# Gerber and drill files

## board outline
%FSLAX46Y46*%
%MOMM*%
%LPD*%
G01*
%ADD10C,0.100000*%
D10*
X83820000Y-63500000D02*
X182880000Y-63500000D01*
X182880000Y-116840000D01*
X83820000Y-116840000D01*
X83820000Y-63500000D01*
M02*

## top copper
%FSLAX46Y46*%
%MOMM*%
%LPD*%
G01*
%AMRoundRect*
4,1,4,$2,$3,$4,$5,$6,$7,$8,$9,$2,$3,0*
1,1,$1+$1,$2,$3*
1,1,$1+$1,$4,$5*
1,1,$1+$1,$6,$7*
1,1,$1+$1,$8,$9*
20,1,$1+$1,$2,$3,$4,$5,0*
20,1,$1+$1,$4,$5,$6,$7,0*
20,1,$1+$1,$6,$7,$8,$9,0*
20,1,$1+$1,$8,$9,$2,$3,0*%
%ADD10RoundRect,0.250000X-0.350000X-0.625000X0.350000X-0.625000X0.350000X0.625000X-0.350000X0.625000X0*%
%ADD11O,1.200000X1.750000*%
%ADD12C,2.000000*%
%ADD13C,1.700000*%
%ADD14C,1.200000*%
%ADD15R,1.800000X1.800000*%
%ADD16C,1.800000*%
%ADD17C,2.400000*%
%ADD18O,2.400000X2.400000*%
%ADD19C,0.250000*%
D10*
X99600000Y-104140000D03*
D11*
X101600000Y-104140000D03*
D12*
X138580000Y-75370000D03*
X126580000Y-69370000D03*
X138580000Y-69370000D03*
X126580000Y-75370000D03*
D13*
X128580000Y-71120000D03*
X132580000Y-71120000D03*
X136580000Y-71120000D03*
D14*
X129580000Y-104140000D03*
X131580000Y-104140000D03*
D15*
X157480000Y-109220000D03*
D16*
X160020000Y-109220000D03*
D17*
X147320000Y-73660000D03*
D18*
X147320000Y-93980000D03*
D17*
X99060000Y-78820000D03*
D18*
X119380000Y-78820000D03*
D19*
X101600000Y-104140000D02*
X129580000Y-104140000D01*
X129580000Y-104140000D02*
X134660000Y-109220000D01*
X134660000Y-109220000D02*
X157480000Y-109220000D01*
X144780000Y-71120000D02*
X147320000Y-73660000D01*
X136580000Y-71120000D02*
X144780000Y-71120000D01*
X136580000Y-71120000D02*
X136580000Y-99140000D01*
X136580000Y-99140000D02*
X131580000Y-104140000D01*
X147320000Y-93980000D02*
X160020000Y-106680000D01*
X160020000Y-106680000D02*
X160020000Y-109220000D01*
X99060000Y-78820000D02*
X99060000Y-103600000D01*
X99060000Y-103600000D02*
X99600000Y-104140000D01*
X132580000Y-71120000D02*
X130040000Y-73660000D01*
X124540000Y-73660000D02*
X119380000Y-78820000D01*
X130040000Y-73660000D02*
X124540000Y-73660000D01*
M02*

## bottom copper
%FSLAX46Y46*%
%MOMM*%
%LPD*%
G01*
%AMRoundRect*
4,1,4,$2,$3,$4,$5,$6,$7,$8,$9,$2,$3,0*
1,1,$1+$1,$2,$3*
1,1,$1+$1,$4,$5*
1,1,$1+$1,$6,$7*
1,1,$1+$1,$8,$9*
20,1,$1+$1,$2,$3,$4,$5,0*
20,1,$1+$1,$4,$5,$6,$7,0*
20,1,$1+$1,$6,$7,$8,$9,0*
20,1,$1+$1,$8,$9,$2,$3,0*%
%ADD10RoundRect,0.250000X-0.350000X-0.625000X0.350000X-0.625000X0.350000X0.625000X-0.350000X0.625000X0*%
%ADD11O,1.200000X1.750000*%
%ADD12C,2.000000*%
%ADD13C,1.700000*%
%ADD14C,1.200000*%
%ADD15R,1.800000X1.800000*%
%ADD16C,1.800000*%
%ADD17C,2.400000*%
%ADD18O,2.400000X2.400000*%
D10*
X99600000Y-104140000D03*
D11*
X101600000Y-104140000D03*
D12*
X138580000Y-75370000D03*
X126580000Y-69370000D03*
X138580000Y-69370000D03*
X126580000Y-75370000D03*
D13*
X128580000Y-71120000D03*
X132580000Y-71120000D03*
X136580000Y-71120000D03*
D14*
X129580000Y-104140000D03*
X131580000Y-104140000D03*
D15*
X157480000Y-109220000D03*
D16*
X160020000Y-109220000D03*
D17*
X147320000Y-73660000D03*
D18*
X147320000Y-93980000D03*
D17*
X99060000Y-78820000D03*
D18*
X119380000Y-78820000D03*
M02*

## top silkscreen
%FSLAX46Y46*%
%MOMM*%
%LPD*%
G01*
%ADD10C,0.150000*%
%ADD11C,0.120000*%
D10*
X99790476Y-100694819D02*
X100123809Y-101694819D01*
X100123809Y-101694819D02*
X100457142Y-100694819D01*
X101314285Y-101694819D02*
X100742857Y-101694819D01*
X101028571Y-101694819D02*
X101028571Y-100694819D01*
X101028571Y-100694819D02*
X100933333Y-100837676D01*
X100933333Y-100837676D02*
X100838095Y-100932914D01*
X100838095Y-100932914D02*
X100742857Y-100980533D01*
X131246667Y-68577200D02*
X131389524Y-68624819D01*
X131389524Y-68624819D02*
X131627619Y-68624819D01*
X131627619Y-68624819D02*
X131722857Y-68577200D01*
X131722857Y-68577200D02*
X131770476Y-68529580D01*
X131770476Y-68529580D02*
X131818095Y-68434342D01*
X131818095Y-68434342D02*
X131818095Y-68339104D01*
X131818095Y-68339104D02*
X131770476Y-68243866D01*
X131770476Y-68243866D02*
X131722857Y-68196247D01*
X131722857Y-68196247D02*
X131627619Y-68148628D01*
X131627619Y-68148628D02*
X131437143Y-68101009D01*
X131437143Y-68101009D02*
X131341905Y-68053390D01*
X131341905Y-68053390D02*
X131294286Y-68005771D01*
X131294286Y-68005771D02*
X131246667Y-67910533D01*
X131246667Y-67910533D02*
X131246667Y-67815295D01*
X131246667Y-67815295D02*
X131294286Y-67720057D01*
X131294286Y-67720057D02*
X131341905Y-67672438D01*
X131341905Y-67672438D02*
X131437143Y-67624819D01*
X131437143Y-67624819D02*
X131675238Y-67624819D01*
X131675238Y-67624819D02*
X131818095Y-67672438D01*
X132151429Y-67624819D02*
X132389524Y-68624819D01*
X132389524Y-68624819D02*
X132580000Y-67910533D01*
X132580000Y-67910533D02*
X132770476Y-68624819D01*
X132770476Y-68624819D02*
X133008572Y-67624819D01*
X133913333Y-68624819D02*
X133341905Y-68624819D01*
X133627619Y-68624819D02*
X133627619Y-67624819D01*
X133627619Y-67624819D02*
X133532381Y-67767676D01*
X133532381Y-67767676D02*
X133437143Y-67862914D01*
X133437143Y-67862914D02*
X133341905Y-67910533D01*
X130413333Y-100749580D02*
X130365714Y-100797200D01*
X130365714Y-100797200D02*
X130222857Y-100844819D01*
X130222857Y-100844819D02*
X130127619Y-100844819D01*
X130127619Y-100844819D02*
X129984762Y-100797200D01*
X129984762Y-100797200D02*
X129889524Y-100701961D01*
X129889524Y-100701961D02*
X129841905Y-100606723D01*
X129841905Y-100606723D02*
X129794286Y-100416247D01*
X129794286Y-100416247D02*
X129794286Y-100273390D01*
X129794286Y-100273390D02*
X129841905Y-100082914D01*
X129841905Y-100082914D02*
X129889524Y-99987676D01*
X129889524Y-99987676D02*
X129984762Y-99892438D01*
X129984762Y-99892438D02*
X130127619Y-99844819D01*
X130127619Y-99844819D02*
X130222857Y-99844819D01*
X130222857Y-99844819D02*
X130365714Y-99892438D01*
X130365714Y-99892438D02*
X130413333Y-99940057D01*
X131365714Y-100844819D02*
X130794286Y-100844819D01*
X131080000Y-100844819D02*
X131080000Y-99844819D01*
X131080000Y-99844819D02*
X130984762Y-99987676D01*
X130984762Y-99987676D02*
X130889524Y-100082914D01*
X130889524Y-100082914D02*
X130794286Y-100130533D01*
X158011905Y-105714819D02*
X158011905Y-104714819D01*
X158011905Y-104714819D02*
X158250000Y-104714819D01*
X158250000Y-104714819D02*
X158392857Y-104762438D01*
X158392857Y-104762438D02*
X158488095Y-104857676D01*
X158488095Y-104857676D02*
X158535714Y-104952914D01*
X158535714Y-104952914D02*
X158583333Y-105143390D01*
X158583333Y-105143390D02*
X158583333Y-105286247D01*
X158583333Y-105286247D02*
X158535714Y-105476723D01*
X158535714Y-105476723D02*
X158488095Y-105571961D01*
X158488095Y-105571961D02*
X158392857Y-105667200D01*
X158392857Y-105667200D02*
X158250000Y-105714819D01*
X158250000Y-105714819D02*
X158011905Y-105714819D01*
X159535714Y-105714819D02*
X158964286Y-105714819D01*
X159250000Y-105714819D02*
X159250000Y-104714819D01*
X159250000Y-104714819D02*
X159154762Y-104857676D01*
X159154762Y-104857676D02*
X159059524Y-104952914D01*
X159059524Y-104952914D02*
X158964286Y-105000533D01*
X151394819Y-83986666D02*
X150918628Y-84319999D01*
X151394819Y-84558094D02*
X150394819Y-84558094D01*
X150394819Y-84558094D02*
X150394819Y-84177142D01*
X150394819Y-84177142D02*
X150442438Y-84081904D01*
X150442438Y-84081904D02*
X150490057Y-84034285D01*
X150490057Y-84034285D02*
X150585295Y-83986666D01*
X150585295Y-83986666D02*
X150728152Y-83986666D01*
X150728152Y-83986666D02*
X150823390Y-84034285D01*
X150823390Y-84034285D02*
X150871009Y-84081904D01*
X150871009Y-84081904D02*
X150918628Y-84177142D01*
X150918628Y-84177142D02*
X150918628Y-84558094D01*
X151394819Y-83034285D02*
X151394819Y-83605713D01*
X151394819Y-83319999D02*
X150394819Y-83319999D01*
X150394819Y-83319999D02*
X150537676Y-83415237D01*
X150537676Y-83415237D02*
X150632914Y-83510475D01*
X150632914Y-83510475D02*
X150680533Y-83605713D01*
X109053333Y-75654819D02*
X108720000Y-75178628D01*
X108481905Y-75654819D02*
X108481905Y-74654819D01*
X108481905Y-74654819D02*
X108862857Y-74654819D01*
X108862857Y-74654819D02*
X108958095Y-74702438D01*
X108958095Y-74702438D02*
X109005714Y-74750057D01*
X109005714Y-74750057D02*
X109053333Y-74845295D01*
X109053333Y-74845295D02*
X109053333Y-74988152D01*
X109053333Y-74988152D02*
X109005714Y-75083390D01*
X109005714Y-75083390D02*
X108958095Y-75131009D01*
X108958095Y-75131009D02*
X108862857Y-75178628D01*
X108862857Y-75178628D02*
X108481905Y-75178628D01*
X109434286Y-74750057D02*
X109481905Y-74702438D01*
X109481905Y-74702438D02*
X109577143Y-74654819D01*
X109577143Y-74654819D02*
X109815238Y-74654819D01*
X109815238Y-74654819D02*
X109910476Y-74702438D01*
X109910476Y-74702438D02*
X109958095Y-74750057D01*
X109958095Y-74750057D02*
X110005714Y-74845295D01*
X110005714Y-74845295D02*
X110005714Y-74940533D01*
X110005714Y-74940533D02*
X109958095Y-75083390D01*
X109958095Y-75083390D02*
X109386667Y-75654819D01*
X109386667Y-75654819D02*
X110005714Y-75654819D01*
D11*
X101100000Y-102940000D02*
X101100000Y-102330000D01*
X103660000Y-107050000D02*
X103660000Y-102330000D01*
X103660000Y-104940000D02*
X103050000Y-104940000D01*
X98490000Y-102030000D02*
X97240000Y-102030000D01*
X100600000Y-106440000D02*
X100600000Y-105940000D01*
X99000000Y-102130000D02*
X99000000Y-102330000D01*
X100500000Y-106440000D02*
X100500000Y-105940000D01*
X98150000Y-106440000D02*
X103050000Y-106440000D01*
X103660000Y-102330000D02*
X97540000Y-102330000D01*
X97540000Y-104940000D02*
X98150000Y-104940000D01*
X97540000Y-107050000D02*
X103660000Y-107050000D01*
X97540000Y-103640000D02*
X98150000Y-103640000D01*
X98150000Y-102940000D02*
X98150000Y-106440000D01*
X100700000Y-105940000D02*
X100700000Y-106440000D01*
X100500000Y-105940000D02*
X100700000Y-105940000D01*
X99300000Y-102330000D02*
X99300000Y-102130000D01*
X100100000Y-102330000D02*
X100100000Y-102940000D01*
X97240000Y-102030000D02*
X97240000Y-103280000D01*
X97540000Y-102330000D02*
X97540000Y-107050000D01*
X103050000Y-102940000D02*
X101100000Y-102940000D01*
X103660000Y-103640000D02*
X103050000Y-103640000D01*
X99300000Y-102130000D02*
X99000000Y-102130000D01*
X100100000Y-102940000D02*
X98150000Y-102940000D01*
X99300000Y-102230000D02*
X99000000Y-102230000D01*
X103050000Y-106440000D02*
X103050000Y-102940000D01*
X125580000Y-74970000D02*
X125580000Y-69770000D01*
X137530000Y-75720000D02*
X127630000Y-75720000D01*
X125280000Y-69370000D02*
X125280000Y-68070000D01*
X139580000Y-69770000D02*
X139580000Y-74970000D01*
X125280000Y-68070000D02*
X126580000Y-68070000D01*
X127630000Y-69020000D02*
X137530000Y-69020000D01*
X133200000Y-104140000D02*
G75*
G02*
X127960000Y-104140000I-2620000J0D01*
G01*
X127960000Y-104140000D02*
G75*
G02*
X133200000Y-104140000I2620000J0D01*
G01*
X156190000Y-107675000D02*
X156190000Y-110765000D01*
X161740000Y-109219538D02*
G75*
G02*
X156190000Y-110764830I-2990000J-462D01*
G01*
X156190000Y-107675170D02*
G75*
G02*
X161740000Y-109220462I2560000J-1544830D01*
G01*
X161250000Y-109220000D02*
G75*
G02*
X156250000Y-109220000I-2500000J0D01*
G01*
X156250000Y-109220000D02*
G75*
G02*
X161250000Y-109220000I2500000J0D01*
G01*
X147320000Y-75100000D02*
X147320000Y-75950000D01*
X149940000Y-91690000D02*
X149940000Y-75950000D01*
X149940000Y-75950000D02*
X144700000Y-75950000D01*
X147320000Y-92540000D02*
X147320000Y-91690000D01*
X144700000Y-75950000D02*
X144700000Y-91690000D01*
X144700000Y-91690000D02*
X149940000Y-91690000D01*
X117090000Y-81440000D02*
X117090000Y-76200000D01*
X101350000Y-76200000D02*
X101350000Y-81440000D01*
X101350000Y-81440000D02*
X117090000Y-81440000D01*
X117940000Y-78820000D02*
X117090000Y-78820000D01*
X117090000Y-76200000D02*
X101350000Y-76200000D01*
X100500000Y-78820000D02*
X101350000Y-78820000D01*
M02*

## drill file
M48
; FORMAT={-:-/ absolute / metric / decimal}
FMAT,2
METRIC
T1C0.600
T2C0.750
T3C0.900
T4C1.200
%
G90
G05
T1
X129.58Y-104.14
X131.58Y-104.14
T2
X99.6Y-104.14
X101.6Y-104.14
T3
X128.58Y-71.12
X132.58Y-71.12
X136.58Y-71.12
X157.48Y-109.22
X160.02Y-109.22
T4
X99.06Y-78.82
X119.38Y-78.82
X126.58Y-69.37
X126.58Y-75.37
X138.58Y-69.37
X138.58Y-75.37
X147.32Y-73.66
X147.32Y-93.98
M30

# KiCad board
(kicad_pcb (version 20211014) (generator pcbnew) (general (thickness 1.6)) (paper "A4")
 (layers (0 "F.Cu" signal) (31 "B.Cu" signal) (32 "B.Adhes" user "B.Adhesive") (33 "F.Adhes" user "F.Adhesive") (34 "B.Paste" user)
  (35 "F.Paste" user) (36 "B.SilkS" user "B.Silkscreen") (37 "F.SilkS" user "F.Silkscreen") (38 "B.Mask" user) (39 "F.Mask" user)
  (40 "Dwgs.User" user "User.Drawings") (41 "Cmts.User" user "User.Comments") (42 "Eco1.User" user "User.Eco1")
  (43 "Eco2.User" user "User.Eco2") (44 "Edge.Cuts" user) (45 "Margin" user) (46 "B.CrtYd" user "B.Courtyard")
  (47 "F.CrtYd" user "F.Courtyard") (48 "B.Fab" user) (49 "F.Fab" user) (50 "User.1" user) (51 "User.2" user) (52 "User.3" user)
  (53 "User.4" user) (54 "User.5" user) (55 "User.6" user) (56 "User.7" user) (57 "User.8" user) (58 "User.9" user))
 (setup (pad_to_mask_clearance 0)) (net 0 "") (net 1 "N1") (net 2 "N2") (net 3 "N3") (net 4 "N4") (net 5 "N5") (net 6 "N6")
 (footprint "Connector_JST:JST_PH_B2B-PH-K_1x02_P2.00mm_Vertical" (layer "F.Cu") (at 99.6 104.14)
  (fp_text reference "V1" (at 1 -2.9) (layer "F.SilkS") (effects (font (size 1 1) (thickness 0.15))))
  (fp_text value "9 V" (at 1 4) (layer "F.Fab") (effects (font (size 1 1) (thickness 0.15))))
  (fp_line (start 1.5 -1.2) (end 1.5 -1.81) (layer "F.SilkS") (width 0.12))
  (fp_line (start 4.06 2.91) (end 4.06 -1.81) (layer "F.SilkS") (width 0.12))
  (fp_line (start 4.06 0.8) (end 3.45 0.8) (layer "F.SilkS") (width 0.12))
  (fp_line (start -1.11 -2.11) (end -2.36 -2.11) (layer "F.SilkS") (width 0.12))
  (fp_line (start 1 2.3) (end 1 1.8) (layer "F.SilkS") (width 0.12))
  (fp_line (start -0.6 -2.01) (end -0.6 -1.81) (layer "F.SilkS") (width 0.12))
  (fp_line (start 0.9 2.3) (end 0.9 1.8) (layer "F.SilkS") (width 0.12))
  (fp_line (start -1.45 2.3) (end 3.45 2.3) (layer "F.SilkS") (width 0.12))
  (fp_line (start 4.06 -1.81) (end -2.06 -1.81) (layer "F.SilkS") (width 0.12))
  (fp_line (start -2.06 0.8) (end -1.45 0.8) (layer "F.SilkS") (width 0.12))
  (fp_line (start -2.06 2.91) (end 4.06 2.91) (layer "F.SilkS") (width 0.12))
  (fp_line (start -2.06 -0.5) (end -1.45 -0.5) (layer "F.SilkS") (width 0.12))
  (fp_line (start -1.45 -1.2) (end -1.45 2.3) (layer "F.SilkS") (width 0.12))
  (fp_line (start 1.1 1.8) (end 1.1 2.3) (layer "F.SilkS") (width 0.12))
  (fp_line (start 0.9 1.8) (end 1.1 1.8) (layer "F.SilkS") (width 0.12))
  (fp_line (start -0.3 -1.81) (end -0.3 -2.01) (layer "F.SilkS") (width 0.12))
  (fp_line (start 0.5 -1.81) (end 0.5 -1.2) (layer "F.SilkS") (width 0.12))
  (fp_line (start -2.36 -2.11) (end -2.36 -0.86) (layer "F.SilkS") (width 0.12))
  (fp_line (start -2.06 -1.81) (end -2.06 2.91) (layer "F.SilkS") (width 0.12))
  (fp_line (start 3.45 -1.2) (end 1.5 -1.2) (layer "F.SilkS") (width 0.12))
  (fp_line (start 4.06 -0.5) (end 3.45 -0.5) (layer "F.SilkS") (width 0.12))
  (fp_line (start -0.3 -2.01) (end -0.6 -2.01) (layer "F.SilkS") (width 0.12))
  (fp_line (start 0.5 -1.2) (end -1.45 -1.2) (layer "F.SilkS") (width 0.12))
  (fp_line (start -0.3 -1.91) (end -0.6 -1.91) (layer "F.SilkS") (width 0.12))
  (fp_line (start 3.45 2.3) (end 3.45 -1.2) (layer "F.SilkS") (width 0.12))
  (pad "1" thru_hole roundrect (at 0 0) (size 1.2 1.75) (drill 0.75) (layers *.Cu *.Mask) (roundrect_rratio 0.208333) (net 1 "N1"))
  (pad "2" thru_hole oval (at 2 0) (size 1.2 1.75) (drill 0.75) (layers *.Cu *.Mask) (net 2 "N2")))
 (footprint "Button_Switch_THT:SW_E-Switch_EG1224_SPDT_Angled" (layer "F.Cu") (at 128.58 71.12)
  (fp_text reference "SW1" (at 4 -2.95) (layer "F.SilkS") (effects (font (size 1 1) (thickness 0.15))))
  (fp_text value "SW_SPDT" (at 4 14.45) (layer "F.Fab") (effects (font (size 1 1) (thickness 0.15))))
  (fp_line (start -3 3.85) (end -3 -1.35) (layer "F.SilkS") (width 0.12))
  (fp_line (start 8.95 4.6) (end -0.95 4.6) (layer "F.SilkS") (width 0.12))
  (fp_line (start -3.3 -1.75) (end -3.3 -3.05) (layer "F.SilkS") (width 0.12))
  (fp_line (start 11 -1.35) (end 11 3.85) (layer "F.SilkS") (width 0.12))
  (fp_line (start -3.3 -3.05) (end -2 -3.05) (layer "F.SilkS") (width 0.12))
  (fp_line (start -0.95 -2.1) (end 8.95 -2.1) (layer "F.SilkS") (width 0.12))
  (pad "" thru_hole circle (at 10 4.25) (size 2 2) (drill 1.2) (layers *.Cu *.Mask))
  (pad "" thru_hole circle (at -2 -1.75) (size 2 2) (drill 1.2) (layers *.Cu *.Mask))
  (pad "" thru_hole circle (at 10 -1.75) (size 2 2) (drill 1.2) (layers *.Cu *.Mask))
  (pad "" thru_hole circle (at -2 4.25) (size 2 2) (drill 1.2) (layers *.Cu *.Mask))
  (pad "1" thru_hole circle (at 0 0) (size 1.7 1.7) (drill 0.9) (layers *.Cu *.Mask) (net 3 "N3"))
  (pad "2" thru_hole circle (at 4 0) (size 1.7 1.7) (drill 0.9) (layers *.Cu *.Mask) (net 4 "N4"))
  (pad "3" thru_hole circle (at 8 0) (size 1.7 1.7) (drill 0.9) (layers *.Cu *.Mask) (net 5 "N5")))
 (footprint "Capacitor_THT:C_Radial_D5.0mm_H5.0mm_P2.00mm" (layer "F.Cu") (at 129.58 104.14)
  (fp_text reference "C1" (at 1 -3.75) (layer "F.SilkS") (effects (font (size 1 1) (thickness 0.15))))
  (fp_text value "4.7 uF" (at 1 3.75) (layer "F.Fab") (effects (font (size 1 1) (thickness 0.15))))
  (fp_circle (center 1 0) (end 3.62 0) (layer "F.SilkS") (width 0.12) (fill none))
  (pad "1" thru_hole circle (at 0 0) (size 1.2 1.2) (drill 0.6) (layers *.Cu *.Mask) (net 2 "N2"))
  (pad "2" thru_hole circle (at 2 0) (size 1.2 1.2) (drill 0.6) (layers *.Cu *.Mask) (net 5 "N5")))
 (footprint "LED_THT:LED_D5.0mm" (layer "F.Cu") (at 157.48 109.22)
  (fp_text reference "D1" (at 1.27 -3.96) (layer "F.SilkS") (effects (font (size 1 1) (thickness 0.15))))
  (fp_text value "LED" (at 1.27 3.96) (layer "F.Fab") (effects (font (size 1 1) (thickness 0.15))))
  (fp_line (start -1.29 -1.545) (end -1.29 1.545) (layer "F.SilkS") (width 0.12))
  (fp_arc (start 4.26 -0.000462) (mid 2.072002 2.880433) (end -1.29 1.54483) (layer "F.SilkS") (width 0.12))
  (fp_arc (start -1.29 -1.54483) (mid 2.072002 -2.880433) (end 4.26 0.000462) (layer "F.SilkS") (width 0.12))
  (fp_circle (center 1.27 0) (end 3.77 0) (layer "F.SilkS") (width 0.12) (fill none))
  (pad "1" thru_hole rect (at 0 0) (size 1.8 1.8) (drill 0.9) (layers *.Cu *.Mask) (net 2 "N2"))
  (pad "2" thru_hole circle (at 2.54 0) (size 1.8 1.8) (drill 0.9) (layers *.Cu *.Mask) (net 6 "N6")))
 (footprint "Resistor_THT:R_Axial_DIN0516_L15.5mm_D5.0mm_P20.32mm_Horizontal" (layer "F.Cu") (at 147.32 73.66 -90)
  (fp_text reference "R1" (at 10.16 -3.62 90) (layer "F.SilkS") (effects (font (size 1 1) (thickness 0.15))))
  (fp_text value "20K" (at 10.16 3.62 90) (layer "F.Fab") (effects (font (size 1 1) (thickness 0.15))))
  (fp_line (start 1.44 0) (end 2.29 0) (layer "F.SilkS") (width 0.12))
  (fp_line (start 18.03 -2.62) (end 2.29 -2.62) (layer "F.SilkS") (width 0.12))
  (fp_line (start 2.29 -2.62) (end 2.29 2.62) (layer "F.SilkS") (width 0.12))
  (fp_line (start 18.88 0) (end 18.03 0) (layer "F.SilkS") (width 0.12))
  (fp_line (start 2.29 2.62) (end 18.03 2.62) (layer "F.SilkS") (width 0.12))
  (fp_line (start 18.03 2.62) (end 18.03 -2.62) (layer "F.SilkS") (width 0.12))
  (pad "1" thru_hole circle (at 0 0 270) (size 2.4 2.4) (drill 1.2) (layers *.Cu *.Mask) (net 5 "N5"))
  (pad "2" thru_hole oval (at 20.32 0 270) (size 2.4 2.4) (drill 1.2) (layers *.Cu *.Mask) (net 6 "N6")))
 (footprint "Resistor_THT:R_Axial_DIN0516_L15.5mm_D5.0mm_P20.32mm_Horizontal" (layer "F.Cu") (at 99.06 78.82)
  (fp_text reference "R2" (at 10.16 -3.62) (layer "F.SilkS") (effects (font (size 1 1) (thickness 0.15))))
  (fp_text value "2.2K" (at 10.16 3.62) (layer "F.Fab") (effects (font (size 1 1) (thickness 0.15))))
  (fp_line (start 18.03 2.62) (end 18.03 -2.62) (layer "F.SilkS") (width 0.12))
  (fp_line (start 2.29 -2.62) (end 2.29 2.62) (layer "F.SilkS") (width 0.12))
  (fp_line (start 2.29 2.62) (end 18.03 2.62) (layer "F.SilkS") (width 0.12))
  (fp_line (start 18.88 0) (end 18.03 0) (layer "F.SilkS") (width 0.12))
  (fp_line (start 18.03 -2.62) (end 2.29 -2.62) (layer "F.SilkS") (width 0.12))
  (fp_line (start 1.44 0) (end 2.29 0) (layer "F.SilkS") (width 0.12))
  (pad "1" thru_hole circle (at 0 0) (size 2.4 2.4) (drill 1.2) (layers *.Cu *.Mask) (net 1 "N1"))
  (pad "2" thru_hole oval (at 20.32 0) (size 2.4 2.4) (drill 1.2) (layers *.Cu *.Mask) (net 4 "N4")))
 (gr_rect (start 182.88 63.5) (end 83.82 116.84) (layer "Edge.Cuts") (width 0.1) (fill none))
 (segment (start 101.6 104.14) (end 129.58 104.14) (width 0.25) (layer "F.Cu") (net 2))
 (segment (start 129.58 104.14) (end 134.66 109.22) (width 0.25) (layer "F.Cu") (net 2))
 (segment (start 134.66 109.22) (end 157.48 109.22) (width 0.25) (layer "F.Cu") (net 2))
 (segment (start 144.78 71.12) (end 147.32 73.66) (width 0.25) (layer "F.Cu") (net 5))
 (segment (start 136.58 71.12) (end 144.78 71.12) (width 0.25) (layer "F.Cu") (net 5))
 (segment (start 136.58 71.12) (end 136.58 99.14) (width 0.25) (layer "F.Cu") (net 5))
 (segment (start 136.58 99.14) (end 131.58 104.14) (width 0.25) (layer "F.Cu") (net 5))
 (segment (start 147.32 93.98) (end 160.02 106.68) (width 0.25) (layer "F.Cu") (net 6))
 (segment (start 160.02 106.68) (end 160.02 109.22) (width 0.25) (layer "F.Cu") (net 6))
 (segment (start 99.06 78.82) (end 99.06 103.6) (width 0.25) (layer "F.Cu") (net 1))
 (segment (start 99.06 103.6) (end 99.6 104.14) (width 0.25) (layer "F.Cu") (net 1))
 (segment (start 132.58 71.12) (end 130.04 73.66) (width 0.25) (layer "F.Cu") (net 4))
 (segment (start 124.54 73.66) (end 119.38 78.82) (width 0.25) (layer "F.Cu") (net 4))
 (segment (start 130.04 73.66) (end 124.54 73.66) (width 0.25) (layer "F.Cu") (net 4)))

